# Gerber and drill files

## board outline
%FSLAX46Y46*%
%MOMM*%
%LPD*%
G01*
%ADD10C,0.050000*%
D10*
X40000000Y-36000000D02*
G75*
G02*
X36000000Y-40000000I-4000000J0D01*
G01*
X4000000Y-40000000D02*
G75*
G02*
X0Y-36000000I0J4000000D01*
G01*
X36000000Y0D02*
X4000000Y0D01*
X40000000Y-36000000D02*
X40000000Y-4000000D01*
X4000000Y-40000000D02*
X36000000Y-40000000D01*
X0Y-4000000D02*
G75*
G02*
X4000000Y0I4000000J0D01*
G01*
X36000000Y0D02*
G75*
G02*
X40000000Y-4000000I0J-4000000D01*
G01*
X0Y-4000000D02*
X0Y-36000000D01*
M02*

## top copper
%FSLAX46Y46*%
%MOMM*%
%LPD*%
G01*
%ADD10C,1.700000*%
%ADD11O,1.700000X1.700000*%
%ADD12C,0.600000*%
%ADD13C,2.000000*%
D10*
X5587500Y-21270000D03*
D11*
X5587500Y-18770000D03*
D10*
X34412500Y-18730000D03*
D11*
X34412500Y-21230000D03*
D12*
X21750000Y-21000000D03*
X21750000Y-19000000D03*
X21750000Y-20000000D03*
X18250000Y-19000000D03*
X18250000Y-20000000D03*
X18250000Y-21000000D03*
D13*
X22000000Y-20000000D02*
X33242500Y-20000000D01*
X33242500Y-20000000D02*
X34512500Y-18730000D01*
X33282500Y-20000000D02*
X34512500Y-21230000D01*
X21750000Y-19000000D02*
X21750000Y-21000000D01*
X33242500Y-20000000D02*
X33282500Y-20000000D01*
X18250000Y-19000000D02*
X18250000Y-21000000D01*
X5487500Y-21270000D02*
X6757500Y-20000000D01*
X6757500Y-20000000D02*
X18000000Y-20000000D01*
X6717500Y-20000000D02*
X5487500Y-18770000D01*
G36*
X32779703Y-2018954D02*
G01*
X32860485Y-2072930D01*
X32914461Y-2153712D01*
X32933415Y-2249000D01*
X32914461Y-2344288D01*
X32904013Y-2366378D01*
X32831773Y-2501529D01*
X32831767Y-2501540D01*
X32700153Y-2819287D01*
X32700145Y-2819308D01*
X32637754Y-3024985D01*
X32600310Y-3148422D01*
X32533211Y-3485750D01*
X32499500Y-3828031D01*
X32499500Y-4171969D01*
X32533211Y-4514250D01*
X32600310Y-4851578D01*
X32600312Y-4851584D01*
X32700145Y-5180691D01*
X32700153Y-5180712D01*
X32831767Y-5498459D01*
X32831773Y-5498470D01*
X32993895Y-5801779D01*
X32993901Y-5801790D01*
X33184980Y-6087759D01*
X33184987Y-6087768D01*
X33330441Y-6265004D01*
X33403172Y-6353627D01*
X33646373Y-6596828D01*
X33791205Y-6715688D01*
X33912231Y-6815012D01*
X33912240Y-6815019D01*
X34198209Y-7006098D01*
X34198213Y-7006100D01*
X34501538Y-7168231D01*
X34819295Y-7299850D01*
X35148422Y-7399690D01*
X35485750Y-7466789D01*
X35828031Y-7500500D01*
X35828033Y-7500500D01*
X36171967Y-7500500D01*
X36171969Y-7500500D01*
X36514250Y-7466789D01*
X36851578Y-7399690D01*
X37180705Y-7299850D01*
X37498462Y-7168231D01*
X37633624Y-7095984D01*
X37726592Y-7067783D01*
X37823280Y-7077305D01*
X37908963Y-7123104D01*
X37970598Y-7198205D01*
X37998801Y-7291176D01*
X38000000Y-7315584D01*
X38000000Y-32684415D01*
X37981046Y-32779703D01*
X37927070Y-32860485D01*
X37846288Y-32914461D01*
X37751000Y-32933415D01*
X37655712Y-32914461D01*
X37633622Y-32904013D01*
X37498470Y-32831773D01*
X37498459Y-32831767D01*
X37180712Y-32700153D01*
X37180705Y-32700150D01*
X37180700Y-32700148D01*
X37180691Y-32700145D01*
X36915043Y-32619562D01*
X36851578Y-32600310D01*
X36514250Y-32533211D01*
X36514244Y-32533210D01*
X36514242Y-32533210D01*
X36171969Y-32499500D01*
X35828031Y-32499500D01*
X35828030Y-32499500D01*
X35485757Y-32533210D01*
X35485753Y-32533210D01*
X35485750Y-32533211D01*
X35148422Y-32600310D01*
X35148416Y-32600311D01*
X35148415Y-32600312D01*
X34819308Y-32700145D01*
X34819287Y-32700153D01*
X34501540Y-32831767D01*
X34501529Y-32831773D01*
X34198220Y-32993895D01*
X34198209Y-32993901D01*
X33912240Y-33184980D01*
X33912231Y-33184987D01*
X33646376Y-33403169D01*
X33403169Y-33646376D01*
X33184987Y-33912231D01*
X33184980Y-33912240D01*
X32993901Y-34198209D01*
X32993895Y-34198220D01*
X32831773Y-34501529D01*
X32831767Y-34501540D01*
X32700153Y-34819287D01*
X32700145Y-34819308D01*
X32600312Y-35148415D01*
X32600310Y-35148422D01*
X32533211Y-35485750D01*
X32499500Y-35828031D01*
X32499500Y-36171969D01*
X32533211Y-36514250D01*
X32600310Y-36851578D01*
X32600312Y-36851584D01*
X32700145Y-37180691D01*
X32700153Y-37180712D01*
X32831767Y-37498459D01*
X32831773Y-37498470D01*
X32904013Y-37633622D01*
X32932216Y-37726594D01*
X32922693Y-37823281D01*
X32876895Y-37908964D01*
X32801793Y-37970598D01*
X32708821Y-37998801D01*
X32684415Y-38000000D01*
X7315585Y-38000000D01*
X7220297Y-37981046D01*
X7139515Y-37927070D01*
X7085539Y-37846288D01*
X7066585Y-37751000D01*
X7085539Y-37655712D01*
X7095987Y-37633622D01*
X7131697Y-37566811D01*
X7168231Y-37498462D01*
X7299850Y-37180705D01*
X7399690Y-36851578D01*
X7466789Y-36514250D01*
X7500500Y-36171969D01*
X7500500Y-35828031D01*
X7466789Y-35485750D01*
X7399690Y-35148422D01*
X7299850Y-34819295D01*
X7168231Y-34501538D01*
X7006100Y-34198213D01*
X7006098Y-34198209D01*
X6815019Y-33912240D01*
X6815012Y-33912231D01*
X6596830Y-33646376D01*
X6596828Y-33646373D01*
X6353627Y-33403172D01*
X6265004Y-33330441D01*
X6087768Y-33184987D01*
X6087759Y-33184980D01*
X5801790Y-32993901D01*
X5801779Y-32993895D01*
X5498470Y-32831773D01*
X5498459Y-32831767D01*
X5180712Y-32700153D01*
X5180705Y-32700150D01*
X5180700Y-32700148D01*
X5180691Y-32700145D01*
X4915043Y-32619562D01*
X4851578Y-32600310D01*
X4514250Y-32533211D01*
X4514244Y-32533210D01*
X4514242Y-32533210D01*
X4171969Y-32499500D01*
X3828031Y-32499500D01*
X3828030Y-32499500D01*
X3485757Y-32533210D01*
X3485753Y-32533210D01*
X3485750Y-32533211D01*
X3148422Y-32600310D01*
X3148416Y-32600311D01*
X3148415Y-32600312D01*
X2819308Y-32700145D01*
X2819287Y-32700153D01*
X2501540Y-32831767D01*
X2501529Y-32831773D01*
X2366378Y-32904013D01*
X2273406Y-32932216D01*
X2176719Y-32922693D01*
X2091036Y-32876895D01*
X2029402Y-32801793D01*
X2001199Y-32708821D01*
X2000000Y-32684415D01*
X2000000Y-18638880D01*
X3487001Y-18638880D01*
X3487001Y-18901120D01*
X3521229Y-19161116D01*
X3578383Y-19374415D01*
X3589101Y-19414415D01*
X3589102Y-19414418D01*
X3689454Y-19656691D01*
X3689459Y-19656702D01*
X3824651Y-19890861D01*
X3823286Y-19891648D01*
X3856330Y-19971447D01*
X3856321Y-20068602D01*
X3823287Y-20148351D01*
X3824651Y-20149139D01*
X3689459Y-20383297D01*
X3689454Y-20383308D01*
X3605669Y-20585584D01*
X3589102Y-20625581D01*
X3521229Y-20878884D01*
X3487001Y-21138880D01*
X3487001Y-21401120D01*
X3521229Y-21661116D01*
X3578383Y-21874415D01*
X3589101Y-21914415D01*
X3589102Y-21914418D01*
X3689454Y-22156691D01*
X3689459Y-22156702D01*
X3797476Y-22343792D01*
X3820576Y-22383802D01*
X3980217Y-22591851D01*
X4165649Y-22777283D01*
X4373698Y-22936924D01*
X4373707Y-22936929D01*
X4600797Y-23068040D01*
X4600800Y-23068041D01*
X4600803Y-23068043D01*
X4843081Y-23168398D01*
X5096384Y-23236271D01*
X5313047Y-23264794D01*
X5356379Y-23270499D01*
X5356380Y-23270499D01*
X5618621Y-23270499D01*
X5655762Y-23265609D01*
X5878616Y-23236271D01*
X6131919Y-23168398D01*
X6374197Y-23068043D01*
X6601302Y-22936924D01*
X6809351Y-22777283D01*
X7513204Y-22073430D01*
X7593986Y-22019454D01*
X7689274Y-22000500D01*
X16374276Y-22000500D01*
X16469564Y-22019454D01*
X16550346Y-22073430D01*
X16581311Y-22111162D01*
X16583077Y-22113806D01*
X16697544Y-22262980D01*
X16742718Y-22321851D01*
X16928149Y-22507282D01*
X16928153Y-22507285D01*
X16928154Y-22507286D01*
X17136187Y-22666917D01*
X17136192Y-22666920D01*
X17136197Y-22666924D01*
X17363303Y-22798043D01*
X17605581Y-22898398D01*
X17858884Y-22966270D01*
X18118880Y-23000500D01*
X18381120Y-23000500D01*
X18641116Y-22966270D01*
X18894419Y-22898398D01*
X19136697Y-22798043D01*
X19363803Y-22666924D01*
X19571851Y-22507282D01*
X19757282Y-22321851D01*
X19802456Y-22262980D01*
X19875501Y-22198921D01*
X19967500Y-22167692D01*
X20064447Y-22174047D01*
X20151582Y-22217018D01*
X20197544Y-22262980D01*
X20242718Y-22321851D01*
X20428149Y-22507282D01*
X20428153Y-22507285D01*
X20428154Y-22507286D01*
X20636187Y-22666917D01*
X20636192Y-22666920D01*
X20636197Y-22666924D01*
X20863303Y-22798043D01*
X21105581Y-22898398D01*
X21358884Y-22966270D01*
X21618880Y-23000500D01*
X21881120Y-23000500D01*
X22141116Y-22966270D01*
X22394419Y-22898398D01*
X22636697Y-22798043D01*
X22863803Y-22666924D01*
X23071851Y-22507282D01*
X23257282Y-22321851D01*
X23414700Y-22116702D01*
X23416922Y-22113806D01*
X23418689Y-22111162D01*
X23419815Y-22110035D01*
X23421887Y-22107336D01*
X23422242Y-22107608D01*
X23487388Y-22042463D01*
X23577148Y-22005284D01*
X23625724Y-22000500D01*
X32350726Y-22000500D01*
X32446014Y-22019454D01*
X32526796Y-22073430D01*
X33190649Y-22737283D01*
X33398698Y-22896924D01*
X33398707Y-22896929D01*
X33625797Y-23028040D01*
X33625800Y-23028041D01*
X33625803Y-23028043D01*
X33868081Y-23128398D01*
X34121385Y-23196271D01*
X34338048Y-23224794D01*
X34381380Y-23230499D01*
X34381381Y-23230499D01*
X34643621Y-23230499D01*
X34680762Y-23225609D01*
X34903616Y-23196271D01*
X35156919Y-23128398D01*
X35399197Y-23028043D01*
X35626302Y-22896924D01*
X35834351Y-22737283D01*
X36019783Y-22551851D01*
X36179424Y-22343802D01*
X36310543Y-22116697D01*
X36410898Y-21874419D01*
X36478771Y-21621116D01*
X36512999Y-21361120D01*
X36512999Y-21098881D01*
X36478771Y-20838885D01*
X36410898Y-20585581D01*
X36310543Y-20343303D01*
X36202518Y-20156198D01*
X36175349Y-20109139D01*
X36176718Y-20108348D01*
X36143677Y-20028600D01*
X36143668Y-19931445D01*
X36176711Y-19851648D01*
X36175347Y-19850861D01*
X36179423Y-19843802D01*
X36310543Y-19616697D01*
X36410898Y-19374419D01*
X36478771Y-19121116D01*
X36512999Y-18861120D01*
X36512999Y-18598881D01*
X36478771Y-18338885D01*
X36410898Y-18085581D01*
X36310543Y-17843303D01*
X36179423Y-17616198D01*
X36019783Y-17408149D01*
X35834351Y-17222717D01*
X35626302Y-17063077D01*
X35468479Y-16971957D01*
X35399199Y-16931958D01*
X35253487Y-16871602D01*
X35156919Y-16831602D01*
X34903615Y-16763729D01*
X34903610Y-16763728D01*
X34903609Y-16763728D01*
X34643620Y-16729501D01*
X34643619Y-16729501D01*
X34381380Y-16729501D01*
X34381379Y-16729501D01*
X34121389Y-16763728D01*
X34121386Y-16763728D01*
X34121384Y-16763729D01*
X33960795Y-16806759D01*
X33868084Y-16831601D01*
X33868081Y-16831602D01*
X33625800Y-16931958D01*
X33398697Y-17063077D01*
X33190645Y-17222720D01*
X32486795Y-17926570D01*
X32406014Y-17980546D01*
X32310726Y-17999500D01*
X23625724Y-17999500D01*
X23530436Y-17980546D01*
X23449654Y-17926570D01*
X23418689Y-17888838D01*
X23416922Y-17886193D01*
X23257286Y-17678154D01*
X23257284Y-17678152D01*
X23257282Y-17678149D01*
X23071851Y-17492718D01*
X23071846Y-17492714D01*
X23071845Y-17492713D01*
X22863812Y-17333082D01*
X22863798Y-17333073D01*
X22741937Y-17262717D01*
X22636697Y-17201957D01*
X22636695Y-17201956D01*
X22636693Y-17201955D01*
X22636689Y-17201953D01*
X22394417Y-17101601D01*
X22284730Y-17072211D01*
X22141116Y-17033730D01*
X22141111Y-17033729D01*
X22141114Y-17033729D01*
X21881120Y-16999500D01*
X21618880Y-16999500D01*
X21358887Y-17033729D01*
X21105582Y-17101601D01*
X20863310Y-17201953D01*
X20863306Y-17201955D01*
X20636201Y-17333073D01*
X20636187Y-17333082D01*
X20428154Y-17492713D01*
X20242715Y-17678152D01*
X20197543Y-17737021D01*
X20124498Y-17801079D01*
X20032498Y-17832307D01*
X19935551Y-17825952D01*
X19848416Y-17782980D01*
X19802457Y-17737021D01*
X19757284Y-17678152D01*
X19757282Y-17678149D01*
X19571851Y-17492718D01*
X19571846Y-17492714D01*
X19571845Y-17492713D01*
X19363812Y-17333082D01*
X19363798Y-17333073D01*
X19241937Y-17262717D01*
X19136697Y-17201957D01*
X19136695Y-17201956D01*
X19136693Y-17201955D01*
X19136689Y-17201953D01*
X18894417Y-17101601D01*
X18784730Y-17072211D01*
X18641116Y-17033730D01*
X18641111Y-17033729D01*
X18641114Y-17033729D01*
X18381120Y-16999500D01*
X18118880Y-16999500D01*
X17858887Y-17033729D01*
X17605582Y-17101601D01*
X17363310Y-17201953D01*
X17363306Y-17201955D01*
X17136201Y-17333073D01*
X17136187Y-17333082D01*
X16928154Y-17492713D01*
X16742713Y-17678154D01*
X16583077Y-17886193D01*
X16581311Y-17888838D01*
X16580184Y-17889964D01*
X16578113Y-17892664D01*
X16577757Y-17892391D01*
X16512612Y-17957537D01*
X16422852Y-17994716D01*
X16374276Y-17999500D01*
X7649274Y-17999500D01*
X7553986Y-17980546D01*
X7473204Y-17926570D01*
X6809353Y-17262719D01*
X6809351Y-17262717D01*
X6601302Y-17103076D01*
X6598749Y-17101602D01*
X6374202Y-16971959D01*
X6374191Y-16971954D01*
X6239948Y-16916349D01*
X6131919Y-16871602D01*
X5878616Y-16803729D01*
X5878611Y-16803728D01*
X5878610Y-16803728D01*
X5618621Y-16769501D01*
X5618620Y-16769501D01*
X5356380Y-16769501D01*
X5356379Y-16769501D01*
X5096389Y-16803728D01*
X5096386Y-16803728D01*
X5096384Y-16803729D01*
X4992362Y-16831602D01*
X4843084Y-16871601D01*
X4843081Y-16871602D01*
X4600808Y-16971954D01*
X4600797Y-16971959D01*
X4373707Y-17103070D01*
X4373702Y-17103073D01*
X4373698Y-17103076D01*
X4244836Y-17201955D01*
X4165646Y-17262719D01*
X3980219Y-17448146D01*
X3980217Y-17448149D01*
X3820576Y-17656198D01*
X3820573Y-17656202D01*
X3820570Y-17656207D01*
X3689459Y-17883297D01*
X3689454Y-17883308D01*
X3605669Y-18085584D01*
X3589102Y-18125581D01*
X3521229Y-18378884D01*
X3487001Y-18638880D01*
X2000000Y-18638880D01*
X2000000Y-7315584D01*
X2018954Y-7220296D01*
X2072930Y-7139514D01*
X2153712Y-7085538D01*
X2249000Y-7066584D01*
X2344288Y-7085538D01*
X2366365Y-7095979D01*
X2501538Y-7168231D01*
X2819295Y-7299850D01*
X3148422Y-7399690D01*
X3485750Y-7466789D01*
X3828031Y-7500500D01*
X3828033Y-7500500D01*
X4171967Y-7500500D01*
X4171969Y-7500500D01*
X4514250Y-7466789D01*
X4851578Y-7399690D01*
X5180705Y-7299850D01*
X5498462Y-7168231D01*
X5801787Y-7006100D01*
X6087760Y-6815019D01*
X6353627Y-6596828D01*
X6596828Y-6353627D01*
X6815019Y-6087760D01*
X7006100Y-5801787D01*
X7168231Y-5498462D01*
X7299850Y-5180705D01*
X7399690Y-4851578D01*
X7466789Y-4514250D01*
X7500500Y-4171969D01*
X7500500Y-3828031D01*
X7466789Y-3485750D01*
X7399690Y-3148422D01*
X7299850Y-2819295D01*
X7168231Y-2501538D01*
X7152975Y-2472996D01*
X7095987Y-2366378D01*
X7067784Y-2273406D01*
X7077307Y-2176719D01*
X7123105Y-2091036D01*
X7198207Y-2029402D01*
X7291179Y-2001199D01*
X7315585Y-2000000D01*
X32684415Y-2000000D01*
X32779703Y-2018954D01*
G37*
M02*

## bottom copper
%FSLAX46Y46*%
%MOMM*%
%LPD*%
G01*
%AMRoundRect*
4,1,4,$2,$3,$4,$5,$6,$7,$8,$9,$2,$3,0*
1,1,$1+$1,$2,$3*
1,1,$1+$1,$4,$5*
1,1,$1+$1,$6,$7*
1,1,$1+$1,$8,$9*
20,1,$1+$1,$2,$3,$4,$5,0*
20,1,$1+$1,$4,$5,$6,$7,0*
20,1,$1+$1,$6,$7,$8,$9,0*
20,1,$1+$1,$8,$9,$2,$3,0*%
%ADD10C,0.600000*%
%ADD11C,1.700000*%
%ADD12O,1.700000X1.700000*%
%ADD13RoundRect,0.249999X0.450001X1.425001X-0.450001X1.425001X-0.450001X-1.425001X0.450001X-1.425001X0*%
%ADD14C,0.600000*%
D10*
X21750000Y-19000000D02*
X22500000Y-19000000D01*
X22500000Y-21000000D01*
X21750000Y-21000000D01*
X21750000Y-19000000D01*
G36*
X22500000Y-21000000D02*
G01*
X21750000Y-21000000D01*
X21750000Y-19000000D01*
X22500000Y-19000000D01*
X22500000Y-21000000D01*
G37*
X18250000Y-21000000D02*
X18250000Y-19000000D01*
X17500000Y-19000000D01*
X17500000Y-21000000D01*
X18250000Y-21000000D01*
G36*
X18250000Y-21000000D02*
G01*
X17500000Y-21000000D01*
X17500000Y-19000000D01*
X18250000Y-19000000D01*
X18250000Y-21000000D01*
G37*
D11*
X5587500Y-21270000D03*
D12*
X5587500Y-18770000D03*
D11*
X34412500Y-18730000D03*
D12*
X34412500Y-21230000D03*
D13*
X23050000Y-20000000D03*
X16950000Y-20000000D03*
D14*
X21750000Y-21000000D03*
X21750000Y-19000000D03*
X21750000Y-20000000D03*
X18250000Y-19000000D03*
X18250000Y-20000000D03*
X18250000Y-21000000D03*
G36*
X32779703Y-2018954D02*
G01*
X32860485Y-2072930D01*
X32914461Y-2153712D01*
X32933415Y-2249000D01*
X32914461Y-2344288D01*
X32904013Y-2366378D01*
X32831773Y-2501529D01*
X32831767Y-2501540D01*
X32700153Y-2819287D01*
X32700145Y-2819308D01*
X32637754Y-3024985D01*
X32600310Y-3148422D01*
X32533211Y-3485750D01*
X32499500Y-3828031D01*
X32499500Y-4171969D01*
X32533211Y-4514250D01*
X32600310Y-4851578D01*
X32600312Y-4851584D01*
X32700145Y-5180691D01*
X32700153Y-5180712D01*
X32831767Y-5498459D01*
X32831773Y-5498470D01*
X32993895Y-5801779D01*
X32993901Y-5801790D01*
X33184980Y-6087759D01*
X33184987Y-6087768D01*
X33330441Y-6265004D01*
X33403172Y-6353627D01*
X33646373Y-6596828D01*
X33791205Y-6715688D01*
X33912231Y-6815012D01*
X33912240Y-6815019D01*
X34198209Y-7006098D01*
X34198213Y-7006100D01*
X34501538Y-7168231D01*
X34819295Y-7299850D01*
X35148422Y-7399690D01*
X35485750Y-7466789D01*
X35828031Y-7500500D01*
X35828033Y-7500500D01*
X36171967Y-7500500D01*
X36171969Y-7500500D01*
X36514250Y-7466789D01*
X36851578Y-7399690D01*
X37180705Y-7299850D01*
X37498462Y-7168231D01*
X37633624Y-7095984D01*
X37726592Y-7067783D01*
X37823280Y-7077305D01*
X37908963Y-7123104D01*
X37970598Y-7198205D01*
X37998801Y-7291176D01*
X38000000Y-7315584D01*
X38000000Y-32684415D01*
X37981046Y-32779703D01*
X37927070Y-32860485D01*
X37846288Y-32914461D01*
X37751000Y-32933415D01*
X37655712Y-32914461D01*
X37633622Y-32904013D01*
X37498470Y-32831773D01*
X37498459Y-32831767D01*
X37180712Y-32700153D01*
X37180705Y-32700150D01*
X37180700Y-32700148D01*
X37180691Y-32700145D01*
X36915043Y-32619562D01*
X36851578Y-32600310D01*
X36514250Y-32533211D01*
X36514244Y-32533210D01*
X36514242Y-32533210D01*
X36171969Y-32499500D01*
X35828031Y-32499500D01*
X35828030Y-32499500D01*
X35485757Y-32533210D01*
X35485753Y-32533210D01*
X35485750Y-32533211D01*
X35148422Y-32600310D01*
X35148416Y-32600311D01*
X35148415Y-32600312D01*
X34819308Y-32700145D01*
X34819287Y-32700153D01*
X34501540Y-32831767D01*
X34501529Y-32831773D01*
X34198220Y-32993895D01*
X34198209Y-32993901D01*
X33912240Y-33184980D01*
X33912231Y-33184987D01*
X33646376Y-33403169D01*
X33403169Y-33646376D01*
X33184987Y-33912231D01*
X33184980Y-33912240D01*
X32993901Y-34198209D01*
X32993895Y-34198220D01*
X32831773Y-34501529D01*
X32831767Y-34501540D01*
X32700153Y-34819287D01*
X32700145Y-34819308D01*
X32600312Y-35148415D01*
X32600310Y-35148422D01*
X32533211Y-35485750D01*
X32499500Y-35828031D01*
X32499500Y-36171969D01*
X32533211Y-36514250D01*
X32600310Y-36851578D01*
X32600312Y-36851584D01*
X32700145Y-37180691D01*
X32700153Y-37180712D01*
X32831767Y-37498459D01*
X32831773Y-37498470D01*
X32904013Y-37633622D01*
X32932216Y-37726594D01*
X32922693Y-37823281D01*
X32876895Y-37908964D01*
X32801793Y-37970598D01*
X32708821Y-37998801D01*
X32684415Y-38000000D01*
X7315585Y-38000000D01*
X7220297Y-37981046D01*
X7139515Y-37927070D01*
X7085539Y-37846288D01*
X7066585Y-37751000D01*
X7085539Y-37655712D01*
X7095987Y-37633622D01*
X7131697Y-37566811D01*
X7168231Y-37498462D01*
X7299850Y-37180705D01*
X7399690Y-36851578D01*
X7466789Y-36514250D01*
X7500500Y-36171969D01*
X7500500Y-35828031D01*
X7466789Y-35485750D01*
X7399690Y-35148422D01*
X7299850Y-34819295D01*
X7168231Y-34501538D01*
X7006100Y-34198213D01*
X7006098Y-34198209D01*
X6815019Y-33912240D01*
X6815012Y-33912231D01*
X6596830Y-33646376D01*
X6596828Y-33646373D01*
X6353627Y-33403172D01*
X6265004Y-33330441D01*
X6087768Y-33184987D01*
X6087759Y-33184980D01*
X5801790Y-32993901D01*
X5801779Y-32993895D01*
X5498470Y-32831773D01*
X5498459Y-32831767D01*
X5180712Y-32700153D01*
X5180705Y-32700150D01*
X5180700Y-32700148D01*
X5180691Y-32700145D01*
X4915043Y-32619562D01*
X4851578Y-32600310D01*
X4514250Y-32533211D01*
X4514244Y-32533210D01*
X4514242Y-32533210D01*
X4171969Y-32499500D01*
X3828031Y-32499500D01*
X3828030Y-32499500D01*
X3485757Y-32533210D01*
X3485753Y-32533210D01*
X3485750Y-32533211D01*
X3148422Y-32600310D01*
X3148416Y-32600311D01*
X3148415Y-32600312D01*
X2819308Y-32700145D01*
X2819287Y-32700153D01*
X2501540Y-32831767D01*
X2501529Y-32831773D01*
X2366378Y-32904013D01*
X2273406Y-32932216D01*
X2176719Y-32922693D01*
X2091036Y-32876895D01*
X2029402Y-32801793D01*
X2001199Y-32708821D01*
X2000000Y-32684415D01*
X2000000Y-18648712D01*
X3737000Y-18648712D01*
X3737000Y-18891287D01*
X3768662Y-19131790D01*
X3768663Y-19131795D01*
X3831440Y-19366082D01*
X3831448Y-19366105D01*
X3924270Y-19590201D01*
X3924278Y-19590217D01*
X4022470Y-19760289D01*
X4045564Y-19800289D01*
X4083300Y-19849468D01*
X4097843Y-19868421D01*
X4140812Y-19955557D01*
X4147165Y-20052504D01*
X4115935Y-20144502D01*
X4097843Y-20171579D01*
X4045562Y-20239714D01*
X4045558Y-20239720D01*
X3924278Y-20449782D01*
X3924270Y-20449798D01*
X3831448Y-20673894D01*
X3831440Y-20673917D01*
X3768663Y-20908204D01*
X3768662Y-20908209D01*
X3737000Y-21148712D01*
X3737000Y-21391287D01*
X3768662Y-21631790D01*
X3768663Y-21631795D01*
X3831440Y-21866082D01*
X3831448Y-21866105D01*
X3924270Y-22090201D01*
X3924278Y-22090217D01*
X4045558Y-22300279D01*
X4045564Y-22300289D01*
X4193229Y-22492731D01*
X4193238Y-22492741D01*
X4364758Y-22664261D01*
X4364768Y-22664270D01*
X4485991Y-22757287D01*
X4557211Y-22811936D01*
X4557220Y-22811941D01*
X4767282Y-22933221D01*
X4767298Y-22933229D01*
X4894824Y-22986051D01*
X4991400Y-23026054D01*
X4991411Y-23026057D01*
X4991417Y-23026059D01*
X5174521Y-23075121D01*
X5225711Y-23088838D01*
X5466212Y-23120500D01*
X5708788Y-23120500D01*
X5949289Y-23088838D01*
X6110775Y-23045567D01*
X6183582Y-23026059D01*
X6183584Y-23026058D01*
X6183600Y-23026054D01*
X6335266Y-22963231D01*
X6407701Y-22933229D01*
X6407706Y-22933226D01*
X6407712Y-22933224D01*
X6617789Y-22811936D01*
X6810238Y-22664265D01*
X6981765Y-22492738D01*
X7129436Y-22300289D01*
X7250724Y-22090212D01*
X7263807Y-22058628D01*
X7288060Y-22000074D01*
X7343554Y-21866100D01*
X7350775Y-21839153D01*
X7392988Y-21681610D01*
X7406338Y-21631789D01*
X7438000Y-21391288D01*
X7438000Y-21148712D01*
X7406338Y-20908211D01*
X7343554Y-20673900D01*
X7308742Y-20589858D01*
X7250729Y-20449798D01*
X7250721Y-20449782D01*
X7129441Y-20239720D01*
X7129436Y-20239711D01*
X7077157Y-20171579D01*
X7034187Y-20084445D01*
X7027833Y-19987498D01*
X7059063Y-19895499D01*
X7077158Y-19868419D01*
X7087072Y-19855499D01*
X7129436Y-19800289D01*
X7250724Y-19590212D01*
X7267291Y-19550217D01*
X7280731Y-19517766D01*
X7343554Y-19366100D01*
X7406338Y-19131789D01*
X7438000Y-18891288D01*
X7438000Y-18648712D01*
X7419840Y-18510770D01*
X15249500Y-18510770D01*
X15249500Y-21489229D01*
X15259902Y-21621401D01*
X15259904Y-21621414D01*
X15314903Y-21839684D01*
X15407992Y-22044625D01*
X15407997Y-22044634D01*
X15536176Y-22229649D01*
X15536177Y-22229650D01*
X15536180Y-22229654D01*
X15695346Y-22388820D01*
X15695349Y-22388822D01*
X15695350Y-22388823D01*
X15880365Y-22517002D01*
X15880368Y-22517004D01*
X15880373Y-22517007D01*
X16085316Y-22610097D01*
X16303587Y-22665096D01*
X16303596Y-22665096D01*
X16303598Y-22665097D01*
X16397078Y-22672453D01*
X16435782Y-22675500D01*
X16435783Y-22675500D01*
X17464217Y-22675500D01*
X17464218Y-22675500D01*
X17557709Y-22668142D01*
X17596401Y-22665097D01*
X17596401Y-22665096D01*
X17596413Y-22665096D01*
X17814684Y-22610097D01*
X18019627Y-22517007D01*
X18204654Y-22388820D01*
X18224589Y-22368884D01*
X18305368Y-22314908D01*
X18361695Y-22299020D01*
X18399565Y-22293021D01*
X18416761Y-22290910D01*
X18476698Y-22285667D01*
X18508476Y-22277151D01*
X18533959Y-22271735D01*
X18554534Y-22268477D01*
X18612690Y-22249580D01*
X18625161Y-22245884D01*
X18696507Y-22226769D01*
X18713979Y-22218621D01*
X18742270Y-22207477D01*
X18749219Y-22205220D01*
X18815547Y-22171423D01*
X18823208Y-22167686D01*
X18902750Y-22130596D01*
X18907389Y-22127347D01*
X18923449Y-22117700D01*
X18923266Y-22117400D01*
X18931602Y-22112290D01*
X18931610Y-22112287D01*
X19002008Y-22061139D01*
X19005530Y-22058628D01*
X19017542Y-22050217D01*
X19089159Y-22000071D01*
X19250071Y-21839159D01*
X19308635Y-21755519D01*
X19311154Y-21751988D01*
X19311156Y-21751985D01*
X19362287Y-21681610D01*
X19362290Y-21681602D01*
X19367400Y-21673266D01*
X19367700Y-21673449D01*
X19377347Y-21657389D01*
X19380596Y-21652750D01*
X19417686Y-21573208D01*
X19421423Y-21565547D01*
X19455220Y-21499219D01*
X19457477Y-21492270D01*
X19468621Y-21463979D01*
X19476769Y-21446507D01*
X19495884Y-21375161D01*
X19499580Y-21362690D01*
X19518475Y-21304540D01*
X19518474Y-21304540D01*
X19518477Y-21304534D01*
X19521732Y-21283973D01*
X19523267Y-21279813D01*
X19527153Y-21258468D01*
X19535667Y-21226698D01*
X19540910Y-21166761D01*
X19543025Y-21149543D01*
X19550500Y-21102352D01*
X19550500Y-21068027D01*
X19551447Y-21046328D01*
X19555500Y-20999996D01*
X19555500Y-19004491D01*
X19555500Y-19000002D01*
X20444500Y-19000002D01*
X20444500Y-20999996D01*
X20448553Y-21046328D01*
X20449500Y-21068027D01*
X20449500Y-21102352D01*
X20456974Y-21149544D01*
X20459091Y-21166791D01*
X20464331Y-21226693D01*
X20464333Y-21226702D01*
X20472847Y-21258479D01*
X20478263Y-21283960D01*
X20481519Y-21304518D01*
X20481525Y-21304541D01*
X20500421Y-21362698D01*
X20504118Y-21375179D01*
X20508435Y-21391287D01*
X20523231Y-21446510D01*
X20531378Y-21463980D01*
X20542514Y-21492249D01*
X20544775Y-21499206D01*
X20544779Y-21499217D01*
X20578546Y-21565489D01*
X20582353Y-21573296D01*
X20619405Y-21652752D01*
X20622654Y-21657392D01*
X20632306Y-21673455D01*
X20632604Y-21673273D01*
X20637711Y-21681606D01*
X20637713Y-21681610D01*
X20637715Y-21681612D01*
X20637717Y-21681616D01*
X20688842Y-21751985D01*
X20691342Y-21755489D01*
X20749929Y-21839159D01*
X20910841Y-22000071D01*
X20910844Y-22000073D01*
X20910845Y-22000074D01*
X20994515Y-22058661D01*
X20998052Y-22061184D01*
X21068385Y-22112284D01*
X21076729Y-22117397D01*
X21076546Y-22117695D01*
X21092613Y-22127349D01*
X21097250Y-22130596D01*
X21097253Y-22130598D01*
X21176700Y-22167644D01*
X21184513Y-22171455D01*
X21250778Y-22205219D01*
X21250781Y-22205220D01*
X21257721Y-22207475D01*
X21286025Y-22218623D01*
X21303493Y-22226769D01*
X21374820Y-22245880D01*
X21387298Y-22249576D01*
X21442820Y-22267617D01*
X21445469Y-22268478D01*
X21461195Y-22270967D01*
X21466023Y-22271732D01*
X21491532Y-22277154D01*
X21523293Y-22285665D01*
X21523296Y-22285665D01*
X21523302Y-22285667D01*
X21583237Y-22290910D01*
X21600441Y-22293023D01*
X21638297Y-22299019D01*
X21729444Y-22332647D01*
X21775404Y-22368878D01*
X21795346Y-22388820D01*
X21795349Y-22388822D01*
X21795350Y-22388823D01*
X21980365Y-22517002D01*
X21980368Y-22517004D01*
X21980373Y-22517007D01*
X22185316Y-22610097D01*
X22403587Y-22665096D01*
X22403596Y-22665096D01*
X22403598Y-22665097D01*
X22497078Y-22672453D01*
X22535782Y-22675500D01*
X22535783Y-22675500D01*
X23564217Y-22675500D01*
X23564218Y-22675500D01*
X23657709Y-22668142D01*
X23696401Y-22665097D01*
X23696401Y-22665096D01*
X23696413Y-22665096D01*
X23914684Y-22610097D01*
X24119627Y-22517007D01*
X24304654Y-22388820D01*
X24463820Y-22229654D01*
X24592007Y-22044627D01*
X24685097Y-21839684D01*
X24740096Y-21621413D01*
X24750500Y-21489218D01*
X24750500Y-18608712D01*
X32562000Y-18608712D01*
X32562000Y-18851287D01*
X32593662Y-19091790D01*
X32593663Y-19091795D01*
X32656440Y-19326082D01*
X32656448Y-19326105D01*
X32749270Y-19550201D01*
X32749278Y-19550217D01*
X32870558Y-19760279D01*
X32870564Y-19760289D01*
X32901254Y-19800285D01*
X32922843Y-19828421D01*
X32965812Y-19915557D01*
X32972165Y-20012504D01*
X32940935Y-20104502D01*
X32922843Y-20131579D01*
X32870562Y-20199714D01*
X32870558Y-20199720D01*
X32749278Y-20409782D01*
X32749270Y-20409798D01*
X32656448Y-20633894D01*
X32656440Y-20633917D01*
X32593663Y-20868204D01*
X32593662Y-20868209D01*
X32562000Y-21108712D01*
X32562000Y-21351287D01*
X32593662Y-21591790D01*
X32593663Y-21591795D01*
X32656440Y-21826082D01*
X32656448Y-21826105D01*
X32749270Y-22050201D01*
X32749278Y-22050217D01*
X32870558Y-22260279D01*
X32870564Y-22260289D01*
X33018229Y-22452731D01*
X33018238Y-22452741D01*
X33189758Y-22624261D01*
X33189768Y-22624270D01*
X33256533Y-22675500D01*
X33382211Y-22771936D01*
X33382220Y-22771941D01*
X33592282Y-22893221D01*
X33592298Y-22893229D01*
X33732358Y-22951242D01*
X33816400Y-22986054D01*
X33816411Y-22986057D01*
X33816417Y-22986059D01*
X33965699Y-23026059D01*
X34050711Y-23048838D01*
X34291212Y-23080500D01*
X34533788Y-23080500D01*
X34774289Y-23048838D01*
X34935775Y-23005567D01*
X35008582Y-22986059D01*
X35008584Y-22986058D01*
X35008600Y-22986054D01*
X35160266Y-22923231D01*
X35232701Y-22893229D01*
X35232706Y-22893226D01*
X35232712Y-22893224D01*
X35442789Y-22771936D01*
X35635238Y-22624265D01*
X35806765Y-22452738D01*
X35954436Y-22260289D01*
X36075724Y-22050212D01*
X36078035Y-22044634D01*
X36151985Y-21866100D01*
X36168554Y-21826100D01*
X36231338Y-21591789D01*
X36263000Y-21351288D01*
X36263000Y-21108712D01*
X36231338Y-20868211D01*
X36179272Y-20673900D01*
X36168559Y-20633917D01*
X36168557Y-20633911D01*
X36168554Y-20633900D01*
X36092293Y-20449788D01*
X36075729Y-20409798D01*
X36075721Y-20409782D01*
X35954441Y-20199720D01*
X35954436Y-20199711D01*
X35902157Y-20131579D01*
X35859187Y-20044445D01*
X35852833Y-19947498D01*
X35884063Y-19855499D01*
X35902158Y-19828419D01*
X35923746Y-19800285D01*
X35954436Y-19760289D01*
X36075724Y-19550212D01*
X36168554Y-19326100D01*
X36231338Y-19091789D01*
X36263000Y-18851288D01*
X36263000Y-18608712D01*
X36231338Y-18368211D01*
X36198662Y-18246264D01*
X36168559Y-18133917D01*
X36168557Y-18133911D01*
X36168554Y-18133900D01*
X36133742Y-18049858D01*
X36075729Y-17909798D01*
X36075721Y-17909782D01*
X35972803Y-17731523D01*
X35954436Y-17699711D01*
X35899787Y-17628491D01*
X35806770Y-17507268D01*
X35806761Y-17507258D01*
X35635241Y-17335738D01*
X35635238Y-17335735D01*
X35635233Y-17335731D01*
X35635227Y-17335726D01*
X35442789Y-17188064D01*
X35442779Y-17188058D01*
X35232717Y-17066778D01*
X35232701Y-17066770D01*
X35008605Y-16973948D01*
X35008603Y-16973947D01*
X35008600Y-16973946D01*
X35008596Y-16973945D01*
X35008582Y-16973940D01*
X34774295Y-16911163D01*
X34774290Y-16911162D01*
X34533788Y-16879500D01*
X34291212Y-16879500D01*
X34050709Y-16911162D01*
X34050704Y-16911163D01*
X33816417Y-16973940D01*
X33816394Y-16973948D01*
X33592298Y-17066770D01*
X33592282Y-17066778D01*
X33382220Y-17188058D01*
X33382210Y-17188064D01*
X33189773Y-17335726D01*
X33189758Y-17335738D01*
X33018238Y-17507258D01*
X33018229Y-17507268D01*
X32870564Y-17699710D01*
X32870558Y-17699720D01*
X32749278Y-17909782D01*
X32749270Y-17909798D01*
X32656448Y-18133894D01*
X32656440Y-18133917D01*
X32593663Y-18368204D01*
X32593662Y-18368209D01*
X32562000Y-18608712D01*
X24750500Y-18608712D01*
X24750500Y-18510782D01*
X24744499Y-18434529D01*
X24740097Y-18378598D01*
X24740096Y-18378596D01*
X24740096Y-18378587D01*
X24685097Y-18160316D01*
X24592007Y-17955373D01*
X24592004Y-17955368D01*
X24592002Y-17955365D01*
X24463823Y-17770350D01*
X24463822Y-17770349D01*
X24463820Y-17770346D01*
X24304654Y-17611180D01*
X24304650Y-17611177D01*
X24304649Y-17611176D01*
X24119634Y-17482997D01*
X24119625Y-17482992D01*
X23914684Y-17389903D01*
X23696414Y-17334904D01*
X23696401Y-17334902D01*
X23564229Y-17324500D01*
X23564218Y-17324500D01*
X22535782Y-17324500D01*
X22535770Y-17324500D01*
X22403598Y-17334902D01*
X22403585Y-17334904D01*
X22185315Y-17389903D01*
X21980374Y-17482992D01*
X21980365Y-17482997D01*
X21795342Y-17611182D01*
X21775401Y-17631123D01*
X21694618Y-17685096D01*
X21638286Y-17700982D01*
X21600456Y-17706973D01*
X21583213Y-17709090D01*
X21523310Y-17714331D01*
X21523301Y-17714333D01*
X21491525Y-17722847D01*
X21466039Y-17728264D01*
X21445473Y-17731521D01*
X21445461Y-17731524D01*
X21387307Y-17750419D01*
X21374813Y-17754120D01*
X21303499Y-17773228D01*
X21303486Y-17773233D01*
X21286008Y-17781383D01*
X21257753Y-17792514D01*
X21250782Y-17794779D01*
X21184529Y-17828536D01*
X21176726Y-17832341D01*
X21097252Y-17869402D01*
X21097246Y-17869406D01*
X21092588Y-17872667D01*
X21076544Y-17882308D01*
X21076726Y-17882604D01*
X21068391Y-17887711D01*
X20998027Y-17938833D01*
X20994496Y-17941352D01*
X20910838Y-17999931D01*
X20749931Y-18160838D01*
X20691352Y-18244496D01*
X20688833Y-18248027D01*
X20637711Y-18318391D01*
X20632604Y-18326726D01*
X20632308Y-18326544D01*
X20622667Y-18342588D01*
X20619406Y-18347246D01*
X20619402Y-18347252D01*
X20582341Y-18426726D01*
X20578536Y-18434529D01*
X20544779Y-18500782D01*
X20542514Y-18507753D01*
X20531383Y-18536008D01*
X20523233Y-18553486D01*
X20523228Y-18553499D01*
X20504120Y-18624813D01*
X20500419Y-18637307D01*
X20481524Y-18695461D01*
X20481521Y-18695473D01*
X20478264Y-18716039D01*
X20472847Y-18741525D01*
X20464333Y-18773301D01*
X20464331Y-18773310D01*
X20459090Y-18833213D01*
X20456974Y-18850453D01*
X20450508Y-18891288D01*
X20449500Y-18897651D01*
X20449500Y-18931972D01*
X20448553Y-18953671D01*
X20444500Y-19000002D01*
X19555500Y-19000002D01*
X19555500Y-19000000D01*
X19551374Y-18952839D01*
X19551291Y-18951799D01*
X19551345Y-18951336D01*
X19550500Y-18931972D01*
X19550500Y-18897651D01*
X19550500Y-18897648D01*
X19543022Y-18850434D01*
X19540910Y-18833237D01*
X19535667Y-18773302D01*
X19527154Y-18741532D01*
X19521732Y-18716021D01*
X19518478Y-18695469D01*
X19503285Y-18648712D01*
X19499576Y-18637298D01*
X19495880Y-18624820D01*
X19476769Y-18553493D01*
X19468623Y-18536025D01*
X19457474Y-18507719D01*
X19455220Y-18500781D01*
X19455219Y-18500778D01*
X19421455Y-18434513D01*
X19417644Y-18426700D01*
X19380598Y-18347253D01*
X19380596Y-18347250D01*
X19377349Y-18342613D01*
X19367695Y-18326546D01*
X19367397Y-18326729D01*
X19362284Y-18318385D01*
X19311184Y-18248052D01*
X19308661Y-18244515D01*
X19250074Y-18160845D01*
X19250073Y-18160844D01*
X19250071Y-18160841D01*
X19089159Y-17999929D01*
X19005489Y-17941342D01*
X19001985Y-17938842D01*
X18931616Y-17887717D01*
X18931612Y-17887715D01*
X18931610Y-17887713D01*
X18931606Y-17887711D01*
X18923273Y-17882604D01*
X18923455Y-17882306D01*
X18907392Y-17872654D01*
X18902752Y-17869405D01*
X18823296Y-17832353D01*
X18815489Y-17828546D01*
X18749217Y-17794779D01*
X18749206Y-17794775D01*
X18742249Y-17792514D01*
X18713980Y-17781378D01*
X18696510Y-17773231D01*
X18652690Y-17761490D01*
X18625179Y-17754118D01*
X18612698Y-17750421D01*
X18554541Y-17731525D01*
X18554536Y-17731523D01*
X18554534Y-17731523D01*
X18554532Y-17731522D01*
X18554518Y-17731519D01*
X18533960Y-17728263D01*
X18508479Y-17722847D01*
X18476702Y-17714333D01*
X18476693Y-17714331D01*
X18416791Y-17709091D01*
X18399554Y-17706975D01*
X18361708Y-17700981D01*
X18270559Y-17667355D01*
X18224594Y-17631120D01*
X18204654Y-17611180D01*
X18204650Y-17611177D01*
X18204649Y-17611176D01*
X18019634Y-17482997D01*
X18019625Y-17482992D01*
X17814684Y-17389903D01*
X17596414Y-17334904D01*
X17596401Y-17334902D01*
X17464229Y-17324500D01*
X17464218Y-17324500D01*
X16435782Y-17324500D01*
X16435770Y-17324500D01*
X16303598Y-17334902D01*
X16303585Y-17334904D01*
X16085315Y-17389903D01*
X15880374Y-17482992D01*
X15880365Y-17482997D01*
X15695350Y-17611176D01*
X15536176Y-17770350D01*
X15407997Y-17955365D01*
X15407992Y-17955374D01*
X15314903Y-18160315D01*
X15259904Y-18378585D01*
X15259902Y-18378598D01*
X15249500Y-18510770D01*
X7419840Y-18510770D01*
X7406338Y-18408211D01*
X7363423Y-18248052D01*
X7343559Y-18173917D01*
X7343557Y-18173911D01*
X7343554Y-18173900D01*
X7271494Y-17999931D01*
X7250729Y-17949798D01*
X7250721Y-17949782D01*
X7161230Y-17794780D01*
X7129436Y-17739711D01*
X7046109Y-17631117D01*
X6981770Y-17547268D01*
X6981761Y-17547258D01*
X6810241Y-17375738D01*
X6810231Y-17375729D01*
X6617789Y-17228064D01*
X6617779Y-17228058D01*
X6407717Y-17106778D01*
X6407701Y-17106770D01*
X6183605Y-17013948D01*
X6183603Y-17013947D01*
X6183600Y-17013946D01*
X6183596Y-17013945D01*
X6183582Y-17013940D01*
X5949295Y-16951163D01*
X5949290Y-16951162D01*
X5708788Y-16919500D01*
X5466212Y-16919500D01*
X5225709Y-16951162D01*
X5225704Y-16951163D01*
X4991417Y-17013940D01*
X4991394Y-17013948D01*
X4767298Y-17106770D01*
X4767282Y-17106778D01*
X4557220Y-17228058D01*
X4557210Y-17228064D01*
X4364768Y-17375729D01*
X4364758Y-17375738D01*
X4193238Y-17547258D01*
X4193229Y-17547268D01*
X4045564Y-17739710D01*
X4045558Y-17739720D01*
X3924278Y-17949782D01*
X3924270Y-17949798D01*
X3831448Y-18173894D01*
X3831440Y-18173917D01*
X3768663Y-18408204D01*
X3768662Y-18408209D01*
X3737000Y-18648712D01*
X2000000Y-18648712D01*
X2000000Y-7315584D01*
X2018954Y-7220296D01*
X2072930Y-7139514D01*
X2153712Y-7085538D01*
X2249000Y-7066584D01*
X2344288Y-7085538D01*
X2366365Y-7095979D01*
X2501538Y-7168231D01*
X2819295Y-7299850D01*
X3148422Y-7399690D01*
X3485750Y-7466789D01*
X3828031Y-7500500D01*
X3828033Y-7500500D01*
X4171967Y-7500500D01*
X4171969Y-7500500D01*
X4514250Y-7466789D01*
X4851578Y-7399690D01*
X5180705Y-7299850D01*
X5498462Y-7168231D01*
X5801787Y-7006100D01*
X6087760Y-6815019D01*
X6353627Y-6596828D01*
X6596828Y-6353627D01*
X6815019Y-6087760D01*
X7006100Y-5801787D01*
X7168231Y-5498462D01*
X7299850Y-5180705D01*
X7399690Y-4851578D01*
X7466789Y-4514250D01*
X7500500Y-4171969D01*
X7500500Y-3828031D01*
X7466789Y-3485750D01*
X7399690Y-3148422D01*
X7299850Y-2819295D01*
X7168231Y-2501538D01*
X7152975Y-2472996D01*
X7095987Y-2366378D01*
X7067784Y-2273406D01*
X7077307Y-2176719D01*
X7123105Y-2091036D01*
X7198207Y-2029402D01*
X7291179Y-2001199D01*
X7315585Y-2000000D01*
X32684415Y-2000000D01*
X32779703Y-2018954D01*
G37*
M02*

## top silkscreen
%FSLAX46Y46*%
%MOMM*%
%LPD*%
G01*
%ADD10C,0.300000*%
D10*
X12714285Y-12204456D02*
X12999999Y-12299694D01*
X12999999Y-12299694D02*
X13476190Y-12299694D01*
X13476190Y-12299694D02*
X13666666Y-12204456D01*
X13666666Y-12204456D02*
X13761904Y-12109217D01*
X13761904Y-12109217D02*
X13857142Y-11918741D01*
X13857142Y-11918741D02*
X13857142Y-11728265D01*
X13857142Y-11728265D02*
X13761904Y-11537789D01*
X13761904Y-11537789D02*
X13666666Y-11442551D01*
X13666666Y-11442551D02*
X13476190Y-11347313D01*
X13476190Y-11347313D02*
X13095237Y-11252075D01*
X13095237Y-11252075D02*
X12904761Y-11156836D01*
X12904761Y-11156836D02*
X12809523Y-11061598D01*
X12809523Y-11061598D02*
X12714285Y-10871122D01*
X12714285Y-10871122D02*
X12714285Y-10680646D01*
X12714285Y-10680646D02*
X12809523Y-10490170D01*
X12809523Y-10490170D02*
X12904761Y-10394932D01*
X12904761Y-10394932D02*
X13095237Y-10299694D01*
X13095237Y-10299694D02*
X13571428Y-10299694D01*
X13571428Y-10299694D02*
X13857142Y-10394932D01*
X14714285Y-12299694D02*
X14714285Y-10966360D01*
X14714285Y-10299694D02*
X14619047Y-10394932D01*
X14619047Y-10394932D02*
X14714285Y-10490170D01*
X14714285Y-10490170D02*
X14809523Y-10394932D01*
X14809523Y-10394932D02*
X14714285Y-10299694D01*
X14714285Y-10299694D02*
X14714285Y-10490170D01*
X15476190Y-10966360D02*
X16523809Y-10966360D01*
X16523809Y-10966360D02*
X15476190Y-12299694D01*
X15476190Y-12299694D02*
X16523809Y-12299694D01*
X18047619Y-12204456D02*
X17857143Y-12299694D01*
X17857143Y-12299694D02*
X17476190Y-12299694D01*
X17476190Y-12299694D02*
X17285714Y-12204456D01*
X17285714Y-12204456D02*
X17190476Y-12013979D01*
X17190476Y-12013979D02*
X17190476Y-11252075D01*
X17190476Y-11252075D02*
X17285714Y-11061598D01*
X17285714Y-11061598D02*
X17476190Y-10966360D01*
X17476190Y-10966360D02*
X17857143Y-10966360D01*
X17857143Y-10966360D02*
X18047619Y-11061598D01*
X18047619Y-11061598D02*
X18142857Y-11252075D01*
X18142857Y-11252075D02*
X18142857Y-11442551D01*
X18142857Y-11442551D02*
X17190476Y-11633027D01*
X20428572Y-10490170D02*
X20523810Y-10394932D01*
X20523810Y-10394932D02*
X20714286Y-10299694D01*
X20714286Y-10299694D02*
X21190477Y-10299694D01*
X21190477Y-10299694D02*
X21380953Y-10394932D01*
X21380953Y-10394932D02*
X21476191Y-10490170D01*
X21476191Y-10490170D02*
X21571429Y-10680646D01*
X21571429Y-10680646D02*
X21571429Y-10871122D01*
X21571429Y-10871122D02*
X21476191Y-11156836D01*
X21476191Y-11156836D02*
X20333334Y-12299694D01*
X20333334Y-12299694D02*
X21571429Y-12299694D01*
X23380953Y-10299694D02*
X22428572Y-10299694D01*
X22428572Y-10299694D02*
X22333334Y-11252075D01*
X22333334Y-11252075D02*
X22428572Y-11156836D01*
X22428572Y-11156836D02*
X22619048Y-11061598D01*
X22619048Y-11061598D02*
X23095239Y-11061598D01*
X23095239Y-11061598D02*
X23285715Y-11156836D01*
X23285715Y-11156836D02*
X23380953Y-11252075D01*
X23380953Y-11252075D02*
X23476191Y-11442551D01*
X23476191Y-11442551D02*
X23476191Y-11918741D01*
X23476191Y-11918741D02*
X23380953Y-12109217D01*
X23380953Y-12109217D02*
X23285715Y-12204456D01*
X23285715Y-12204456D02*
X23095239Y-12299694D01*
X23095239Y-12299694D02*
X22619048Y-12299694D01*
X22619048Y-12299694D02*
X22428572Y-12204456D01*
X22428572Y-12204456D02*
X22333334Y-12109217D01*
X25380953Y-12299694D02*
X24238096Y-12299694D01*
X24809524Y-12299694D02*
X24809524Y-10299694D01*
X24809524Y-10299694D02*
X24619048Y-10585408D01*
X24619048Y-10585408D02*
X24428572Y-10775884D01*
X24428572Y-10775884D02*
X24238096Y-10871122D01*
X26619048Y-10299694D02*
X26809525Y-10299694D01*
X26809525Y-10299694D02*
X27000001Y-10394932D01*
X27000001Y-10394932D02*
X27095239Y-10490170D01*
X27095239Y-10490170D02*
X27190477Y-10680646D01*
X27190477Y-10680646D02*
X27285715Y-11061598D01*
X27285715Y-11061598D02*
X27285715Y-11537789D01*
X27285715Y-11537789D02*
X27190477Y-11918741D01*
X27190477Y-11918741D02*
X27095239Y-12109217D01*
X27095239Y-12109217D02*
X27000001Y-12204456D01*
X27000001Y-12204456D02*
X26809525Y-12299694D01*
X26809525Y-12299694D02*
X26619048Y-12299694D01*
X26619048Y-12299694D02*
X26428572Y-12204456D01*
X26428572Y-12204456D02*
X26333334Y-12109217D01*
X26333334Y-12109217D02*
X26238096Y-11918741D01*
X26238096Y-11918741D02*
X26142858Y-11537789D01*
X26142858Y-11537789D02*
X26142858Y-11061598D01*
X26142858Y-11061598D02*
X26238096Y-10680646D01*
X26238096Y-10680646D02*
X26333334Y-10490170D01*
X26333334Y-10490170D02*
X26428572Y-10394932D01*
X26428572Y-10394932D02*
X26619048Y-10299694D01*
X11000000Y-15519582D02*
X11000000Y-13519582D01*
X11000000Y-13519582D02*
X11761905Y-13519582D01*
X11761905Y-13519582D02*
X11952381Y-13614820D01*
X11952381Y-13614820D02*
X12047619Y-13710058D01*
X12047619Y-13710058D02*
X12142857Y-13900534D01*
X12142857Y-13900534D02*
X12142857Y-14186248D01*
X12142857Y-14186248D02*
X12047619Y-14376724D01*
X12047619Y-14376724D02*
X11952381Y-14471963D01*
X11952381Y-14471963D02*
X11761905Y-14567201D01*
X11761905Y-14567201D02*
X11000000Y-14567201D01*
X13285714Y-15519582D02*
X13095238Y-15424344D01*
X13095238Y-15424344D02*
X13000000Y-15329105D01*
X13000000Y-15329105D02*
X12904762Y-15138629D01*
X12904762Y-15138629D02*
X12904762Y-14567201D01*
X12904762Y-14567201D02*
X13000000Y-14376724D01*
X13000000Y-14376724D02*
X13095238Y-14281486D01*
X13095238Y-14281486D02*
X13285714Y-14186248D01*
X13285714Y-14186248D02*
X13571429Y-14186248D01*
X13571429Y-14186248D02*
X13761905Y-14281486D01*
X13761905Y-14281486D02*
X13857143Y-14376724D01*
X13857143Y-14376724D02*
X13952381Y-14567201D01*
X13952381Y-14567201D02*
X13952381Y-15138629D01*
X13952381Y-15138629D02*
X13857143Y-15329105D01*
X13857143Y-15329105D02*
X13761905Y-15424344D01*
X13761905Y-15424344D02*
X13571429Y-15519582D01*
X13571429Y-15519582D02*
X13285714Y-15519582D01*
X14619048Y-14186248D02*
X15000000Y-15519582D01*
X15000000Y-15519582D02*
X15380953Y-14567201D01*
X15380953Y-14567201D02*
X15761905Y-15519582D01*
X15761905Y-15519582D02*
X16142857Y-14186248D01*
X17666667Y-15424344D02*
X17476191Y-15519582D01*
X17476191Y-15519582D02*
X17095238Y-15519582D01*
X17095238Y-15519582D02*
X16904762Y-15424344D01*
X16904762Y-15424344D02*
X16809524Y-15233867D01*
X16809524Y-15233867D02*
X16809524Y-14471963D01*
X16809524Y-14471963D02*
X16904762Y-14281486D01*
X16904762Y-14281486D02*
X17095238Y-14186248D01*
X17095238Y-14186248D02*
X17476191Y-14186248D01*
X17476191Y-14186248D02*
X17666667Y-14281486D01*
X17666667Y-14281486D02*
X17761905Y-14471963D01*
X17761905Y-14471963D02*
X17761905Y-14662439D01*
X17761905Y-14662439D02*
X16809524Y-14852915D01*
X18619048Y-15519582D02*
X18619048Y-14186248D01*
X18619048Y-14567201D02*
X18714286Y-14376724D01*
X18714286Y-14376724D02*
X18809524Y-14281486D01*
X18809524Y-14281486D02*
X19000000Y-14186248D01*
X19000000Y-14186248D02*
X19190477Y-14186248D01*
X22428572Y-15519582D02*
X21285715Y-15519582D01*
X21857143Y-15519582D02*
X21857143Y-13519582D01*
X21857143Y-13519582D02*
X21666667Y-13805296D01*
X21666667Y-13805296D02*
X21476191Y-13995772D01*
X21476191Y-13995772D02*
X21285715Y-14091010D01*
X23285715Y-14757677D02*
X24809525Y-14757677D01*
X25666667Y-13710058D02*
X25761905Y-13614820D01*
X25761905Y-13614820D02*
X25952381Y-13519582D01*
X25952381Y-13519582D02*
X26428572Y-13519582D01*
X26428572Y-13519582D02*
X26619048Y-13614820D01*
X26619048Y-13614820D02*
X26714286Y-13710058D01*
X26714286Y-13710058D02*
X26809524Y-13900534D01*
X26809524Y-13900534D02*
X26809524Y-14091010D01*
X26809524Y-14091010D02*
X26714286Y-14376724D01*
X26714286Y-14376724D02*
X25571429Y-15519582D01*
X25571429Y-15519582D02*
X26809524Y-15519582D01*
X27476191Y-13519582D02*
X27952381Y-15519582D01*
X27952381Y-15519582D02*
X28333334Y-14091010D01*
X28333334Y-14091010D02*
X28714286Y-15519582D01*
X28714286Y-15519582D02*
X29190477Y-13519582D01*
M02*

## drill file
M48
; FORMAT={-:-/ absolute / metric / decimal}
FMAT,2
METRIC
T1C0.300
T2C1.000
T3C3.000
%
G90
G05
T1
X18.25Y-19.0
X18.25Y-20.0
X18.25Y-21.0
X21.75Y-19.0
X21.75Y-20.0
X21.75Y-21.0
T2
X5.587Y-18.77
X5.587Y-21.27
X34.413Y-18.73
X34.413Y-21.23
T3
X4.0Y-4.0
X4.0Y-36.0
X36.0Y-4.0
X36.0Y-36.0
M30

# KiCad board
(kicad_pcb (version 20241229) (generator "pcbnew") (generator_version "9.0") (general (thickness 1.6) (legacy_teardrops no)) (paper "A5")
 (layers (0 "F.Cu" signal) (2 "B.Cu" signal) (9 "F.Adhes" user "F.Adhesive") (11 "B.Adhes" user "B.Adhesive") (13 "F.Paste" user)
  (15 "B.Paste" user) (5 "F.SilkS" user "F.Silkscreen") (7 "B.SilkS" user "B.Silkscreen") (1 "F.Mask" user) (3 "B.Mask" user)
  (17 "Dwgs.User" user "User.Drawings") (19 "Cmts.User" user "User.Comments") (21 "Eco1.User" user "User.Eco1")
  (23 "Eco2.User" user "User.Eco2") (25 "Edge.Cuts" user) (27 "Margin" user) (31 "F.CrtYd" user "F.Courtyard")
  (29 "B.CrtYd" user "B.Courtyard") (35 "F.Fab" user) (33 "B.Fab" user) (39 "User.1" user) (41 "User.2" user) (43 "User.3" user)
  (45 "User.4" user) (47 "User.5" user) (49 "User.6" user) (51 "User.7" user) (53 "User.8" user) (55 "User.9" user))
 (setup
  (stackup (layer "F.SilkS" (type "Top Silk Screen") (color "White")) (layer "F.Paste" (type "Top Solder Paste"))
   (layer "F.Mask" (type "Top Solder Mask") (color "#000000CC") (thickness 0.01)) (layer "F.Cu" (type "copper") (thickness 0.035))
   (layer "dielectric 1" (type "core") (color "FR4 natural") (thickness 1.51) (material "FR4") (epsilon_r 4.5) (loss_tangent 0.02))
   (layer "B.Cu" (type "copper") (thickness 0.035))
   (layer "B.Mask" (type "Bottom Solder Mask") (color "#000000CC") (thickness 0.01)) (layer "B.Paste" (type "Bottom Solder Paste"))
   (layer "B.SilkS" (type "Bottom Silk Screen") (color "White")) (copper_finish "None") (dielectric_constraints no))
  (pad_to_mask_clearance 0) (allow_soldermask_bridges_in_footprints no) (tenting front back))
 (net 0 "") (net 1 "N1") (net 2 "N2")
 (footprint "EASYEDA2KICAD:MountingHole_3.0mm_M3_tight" (layer "F.Cu") (at 36 36 -90)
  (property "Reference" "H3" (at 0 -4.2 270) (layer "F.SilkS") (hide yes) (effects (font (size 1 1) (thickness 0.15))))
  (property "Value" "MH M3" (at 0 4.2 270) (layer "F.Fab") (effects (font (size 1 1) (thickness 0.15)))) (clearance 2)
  (pad "" np_thru_hole circle (at 0 0 270) (size 3 3) (drill 3) (layers "*.Cu" "*.Mask")))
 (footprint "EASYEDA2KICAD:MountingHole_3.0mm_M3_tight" (layer "F.Cu") (at 36 4 -90)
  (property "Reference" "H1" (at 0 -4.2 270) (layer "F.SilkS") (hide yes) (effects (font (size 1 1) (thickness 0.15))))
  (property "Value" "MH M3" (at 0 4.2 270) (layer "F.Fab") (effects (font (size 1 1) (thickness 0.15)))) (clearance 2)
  (pad "" np_thru_hole circle (at 0 0 270) (size 3 3) (drill 3) (layers "*.Cu" "*.Mask")))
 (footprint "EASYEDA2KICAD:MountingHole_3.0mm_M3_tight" (layer "F.Cu") (at 4 36 -90)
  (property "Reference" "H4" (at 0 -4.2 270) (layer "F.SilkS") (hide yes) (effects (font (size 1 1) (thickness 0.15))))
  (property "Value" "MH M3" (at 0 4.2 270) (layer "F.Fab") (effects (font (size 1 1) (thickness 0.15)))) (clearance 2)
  (pad "" np_thru_hole circle (at 0 0 270) (size 3 3) (drill 3) (layers "*.Cu" "*.Mask")))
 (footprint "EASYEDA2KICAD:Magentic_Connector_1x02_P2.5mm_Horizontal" (layer "F.Cu") (at 5.4875 20 180)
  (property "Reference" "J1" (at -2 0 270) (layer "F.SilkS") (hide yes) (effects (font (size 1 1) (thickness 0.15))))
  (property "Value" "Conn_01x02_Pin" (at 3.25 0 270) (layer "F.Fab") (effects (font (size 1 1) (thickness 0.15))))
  (pad "1" thru_hole circle (at -0.1 -1.27 180) (size 1.7 1.7) (drill 1) (layers "*.Cu" "*.Mask") (remove_unused_layers no) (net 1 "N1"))
  (pad "2" thru_hole oval (at -0.1 1.23 180) (size 1.7 1.7) (drill 1) (layers "*.Cu" "*.Mask") (remove_unused_layers no) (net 1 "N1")))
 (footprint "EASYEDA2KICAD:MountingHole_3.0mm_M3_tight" (layer "F.Cu") (at 4 4 -90)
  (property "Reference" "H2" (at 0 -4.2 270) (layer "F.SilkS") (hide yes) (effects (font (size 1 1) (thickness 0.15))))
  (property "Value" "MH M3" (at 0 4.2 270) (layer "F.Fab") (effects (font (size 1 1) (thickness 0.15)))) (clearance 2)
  (pad "" np_thru_hole circle (at 0 0 270) (size 3 3) (drill 3) (layers "*.Cu" "*.Mask")))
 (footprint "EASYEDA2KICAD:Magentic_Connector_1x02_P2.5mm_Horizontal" (layer "F.Cu") (at 34.5125 20)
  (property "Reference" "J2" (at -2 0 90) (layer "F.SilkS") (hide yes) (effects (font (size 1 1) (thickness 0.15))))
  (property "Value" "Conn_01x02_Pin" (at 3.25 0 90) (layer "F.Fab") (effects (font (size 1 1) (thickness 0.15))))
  (pad "1" thru_hole circle (at -0.1 -1.27) (size 1.7 1.7) (drill 1) (layers "*.Cu" "*.Mask") (remove_unused_layers no) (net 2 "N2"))
  (pad "2" thru_hole oval (at -0.1 1.23) (size 1.7 1.7) (drill 1) (layers "*.Cu" "*.Mask") (remove_unused_layers no) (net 2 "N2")))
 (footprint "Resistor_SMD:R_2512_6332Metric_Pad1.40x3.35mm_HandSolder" (layer "B.Cu") (at 20 20 180)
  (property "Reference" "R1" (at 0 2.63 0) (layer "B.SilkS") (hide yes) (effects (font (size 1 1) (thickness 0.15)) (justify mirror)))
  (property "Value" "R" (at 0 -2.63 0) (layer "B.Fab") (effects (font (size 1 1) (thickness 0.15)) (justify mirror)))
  (pad "1" smd roundrect (at -3.05 0 180) (size 1.4 3.35) (layers "B.Cu" "B.Mask" "B.Paste") (roundrect_rratio 0.178571) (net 2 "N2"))
  (pad "2" smd roundrect (at 3.05 0 180) (size 1.4 3.35) (layers "B.Cu" "B.Mask" "B.Paste") (roundrect_rratio 0.178571) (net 1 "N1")))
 (gr_poly (pts (xy 21.75 19) (xy 22.5 19) (xy 22.5 21) (xy 21.75 21)) (stroke (width 0.6) (type solid)) (fill yes) (layer "B.Cu") (net 2))
 (gr_poly (pts (xy 18.25 21) (xy 18.25 19) (xy 17.5 19) (xy 17.5 21)) (stroke (width 0.6) (type solid)) (fill yes) (layer "B.Cu") (net 1))
 (gr_arc (start 40 36) (mid 38.828427 38.828427) (end 36 40) (stroke (width 0.05) (type default)) (layer "Edge.Cuts"))
 (gr_arc (start 4 40) (mid 1.171573 38.828427) (end 0 36) (stroke (width 0.05) (type default)) (layer "Edge.Cuts"))
 (gr_line (start 36 0) (end 4 0) (stroke (width 0.05) (type default)) (layer "Edge.Cuts"))
 (gr_line (start 40 36) (end 40 4) (stroke (width 0.05) (type default)) (layer "Edge.Cuts"))
 (gr_line (start 4 40) (end 36 40) (stroke (width 0.05) (type default)) (layer "Edge.Cuts"))
 (gr_arc (start 0 4) (mid 1.171573 1.171573) (end 4 0) (stroke (width 0.05) (type default)) (layer "Edge.Cuts"))
 (gr_arc (start 36 0) (mid 38.828427 1.171573) (end 40 4) (stroke (width 0.05) (type default)) (layer "Edge.Cuts"))
 (gr_line (start 0 4) (end 0 36) (stroke (width 0.05) (type default)) (layer "Edge.Cuts"))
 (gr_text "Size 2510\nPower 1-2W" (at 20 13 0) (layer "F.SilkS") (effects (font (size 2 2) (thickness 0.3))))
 (segment (start 22 20) (end 33.2425 20) (width 2) (layer "F.Cu") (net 2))
 (segment (start 33.2425 20) (end 34.5125 18.73) (width 2) (layer "F.Cu") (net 2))
 (segment (start 33.2825 20) (end 34.5125 21.23) (width 2) (layer "F.Cu") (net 2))
 (segment (start 21.75 19) (end 21.75 21) (width 2) (layer "F.Cu") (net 2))
 (segment (start 33.2425 20) (end 33.2825 20) (width 2) (layer "F.Cu") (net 2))
 (via (at 21.75 21) (size 0.6) (drill 0.3) (layers "F.Cu" "B.Cu") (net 2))
 (via (at 21.75 19) (size 0.6) (drill 0.3) (layers "F.Cu" "B.Cu") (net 2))
 (via (at 21.75 20) (size 0.6) (drill 0.3) (layers "F.Cu" "B.Cu") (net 2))
 (segment (start 18.25 19) (end 18.25 21) (width 2) (layer "F.Cu") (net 1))
 (segment (start 5.4875 21.27) (end 6.7575 20) (width 2) (layer "F.Cu") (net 1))
 (segment (start 6.7575 20) (end 18 20) (width 2) (layer "F.Cu") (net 1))
 (segment (start 6.7175 20) (end 5.4875 18.77) (width 2) (layer "F.Cu") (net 1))
 (via (at 18.25 19) (size 0.6) (drill 0.3) (layers "F.Cu" "B.Cu") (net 1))
 (via (at 18.25 20) (size 0.6) (drill 0.3) (layers "F.Cu" "B.Cu") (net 1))
 (via (at 18.25 21) (size 0.6) (drill 0.3) (layers "F.Cu" "B.Cu") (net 1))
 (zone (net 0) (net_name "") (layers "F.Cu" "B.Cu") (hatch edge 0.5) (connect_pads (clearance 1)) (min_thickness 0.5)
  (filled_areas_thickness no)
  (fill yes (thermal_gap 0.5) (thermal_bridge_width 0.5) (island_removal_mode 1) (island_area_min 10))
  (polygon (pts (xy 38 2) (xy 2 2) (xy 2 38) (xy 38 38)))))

